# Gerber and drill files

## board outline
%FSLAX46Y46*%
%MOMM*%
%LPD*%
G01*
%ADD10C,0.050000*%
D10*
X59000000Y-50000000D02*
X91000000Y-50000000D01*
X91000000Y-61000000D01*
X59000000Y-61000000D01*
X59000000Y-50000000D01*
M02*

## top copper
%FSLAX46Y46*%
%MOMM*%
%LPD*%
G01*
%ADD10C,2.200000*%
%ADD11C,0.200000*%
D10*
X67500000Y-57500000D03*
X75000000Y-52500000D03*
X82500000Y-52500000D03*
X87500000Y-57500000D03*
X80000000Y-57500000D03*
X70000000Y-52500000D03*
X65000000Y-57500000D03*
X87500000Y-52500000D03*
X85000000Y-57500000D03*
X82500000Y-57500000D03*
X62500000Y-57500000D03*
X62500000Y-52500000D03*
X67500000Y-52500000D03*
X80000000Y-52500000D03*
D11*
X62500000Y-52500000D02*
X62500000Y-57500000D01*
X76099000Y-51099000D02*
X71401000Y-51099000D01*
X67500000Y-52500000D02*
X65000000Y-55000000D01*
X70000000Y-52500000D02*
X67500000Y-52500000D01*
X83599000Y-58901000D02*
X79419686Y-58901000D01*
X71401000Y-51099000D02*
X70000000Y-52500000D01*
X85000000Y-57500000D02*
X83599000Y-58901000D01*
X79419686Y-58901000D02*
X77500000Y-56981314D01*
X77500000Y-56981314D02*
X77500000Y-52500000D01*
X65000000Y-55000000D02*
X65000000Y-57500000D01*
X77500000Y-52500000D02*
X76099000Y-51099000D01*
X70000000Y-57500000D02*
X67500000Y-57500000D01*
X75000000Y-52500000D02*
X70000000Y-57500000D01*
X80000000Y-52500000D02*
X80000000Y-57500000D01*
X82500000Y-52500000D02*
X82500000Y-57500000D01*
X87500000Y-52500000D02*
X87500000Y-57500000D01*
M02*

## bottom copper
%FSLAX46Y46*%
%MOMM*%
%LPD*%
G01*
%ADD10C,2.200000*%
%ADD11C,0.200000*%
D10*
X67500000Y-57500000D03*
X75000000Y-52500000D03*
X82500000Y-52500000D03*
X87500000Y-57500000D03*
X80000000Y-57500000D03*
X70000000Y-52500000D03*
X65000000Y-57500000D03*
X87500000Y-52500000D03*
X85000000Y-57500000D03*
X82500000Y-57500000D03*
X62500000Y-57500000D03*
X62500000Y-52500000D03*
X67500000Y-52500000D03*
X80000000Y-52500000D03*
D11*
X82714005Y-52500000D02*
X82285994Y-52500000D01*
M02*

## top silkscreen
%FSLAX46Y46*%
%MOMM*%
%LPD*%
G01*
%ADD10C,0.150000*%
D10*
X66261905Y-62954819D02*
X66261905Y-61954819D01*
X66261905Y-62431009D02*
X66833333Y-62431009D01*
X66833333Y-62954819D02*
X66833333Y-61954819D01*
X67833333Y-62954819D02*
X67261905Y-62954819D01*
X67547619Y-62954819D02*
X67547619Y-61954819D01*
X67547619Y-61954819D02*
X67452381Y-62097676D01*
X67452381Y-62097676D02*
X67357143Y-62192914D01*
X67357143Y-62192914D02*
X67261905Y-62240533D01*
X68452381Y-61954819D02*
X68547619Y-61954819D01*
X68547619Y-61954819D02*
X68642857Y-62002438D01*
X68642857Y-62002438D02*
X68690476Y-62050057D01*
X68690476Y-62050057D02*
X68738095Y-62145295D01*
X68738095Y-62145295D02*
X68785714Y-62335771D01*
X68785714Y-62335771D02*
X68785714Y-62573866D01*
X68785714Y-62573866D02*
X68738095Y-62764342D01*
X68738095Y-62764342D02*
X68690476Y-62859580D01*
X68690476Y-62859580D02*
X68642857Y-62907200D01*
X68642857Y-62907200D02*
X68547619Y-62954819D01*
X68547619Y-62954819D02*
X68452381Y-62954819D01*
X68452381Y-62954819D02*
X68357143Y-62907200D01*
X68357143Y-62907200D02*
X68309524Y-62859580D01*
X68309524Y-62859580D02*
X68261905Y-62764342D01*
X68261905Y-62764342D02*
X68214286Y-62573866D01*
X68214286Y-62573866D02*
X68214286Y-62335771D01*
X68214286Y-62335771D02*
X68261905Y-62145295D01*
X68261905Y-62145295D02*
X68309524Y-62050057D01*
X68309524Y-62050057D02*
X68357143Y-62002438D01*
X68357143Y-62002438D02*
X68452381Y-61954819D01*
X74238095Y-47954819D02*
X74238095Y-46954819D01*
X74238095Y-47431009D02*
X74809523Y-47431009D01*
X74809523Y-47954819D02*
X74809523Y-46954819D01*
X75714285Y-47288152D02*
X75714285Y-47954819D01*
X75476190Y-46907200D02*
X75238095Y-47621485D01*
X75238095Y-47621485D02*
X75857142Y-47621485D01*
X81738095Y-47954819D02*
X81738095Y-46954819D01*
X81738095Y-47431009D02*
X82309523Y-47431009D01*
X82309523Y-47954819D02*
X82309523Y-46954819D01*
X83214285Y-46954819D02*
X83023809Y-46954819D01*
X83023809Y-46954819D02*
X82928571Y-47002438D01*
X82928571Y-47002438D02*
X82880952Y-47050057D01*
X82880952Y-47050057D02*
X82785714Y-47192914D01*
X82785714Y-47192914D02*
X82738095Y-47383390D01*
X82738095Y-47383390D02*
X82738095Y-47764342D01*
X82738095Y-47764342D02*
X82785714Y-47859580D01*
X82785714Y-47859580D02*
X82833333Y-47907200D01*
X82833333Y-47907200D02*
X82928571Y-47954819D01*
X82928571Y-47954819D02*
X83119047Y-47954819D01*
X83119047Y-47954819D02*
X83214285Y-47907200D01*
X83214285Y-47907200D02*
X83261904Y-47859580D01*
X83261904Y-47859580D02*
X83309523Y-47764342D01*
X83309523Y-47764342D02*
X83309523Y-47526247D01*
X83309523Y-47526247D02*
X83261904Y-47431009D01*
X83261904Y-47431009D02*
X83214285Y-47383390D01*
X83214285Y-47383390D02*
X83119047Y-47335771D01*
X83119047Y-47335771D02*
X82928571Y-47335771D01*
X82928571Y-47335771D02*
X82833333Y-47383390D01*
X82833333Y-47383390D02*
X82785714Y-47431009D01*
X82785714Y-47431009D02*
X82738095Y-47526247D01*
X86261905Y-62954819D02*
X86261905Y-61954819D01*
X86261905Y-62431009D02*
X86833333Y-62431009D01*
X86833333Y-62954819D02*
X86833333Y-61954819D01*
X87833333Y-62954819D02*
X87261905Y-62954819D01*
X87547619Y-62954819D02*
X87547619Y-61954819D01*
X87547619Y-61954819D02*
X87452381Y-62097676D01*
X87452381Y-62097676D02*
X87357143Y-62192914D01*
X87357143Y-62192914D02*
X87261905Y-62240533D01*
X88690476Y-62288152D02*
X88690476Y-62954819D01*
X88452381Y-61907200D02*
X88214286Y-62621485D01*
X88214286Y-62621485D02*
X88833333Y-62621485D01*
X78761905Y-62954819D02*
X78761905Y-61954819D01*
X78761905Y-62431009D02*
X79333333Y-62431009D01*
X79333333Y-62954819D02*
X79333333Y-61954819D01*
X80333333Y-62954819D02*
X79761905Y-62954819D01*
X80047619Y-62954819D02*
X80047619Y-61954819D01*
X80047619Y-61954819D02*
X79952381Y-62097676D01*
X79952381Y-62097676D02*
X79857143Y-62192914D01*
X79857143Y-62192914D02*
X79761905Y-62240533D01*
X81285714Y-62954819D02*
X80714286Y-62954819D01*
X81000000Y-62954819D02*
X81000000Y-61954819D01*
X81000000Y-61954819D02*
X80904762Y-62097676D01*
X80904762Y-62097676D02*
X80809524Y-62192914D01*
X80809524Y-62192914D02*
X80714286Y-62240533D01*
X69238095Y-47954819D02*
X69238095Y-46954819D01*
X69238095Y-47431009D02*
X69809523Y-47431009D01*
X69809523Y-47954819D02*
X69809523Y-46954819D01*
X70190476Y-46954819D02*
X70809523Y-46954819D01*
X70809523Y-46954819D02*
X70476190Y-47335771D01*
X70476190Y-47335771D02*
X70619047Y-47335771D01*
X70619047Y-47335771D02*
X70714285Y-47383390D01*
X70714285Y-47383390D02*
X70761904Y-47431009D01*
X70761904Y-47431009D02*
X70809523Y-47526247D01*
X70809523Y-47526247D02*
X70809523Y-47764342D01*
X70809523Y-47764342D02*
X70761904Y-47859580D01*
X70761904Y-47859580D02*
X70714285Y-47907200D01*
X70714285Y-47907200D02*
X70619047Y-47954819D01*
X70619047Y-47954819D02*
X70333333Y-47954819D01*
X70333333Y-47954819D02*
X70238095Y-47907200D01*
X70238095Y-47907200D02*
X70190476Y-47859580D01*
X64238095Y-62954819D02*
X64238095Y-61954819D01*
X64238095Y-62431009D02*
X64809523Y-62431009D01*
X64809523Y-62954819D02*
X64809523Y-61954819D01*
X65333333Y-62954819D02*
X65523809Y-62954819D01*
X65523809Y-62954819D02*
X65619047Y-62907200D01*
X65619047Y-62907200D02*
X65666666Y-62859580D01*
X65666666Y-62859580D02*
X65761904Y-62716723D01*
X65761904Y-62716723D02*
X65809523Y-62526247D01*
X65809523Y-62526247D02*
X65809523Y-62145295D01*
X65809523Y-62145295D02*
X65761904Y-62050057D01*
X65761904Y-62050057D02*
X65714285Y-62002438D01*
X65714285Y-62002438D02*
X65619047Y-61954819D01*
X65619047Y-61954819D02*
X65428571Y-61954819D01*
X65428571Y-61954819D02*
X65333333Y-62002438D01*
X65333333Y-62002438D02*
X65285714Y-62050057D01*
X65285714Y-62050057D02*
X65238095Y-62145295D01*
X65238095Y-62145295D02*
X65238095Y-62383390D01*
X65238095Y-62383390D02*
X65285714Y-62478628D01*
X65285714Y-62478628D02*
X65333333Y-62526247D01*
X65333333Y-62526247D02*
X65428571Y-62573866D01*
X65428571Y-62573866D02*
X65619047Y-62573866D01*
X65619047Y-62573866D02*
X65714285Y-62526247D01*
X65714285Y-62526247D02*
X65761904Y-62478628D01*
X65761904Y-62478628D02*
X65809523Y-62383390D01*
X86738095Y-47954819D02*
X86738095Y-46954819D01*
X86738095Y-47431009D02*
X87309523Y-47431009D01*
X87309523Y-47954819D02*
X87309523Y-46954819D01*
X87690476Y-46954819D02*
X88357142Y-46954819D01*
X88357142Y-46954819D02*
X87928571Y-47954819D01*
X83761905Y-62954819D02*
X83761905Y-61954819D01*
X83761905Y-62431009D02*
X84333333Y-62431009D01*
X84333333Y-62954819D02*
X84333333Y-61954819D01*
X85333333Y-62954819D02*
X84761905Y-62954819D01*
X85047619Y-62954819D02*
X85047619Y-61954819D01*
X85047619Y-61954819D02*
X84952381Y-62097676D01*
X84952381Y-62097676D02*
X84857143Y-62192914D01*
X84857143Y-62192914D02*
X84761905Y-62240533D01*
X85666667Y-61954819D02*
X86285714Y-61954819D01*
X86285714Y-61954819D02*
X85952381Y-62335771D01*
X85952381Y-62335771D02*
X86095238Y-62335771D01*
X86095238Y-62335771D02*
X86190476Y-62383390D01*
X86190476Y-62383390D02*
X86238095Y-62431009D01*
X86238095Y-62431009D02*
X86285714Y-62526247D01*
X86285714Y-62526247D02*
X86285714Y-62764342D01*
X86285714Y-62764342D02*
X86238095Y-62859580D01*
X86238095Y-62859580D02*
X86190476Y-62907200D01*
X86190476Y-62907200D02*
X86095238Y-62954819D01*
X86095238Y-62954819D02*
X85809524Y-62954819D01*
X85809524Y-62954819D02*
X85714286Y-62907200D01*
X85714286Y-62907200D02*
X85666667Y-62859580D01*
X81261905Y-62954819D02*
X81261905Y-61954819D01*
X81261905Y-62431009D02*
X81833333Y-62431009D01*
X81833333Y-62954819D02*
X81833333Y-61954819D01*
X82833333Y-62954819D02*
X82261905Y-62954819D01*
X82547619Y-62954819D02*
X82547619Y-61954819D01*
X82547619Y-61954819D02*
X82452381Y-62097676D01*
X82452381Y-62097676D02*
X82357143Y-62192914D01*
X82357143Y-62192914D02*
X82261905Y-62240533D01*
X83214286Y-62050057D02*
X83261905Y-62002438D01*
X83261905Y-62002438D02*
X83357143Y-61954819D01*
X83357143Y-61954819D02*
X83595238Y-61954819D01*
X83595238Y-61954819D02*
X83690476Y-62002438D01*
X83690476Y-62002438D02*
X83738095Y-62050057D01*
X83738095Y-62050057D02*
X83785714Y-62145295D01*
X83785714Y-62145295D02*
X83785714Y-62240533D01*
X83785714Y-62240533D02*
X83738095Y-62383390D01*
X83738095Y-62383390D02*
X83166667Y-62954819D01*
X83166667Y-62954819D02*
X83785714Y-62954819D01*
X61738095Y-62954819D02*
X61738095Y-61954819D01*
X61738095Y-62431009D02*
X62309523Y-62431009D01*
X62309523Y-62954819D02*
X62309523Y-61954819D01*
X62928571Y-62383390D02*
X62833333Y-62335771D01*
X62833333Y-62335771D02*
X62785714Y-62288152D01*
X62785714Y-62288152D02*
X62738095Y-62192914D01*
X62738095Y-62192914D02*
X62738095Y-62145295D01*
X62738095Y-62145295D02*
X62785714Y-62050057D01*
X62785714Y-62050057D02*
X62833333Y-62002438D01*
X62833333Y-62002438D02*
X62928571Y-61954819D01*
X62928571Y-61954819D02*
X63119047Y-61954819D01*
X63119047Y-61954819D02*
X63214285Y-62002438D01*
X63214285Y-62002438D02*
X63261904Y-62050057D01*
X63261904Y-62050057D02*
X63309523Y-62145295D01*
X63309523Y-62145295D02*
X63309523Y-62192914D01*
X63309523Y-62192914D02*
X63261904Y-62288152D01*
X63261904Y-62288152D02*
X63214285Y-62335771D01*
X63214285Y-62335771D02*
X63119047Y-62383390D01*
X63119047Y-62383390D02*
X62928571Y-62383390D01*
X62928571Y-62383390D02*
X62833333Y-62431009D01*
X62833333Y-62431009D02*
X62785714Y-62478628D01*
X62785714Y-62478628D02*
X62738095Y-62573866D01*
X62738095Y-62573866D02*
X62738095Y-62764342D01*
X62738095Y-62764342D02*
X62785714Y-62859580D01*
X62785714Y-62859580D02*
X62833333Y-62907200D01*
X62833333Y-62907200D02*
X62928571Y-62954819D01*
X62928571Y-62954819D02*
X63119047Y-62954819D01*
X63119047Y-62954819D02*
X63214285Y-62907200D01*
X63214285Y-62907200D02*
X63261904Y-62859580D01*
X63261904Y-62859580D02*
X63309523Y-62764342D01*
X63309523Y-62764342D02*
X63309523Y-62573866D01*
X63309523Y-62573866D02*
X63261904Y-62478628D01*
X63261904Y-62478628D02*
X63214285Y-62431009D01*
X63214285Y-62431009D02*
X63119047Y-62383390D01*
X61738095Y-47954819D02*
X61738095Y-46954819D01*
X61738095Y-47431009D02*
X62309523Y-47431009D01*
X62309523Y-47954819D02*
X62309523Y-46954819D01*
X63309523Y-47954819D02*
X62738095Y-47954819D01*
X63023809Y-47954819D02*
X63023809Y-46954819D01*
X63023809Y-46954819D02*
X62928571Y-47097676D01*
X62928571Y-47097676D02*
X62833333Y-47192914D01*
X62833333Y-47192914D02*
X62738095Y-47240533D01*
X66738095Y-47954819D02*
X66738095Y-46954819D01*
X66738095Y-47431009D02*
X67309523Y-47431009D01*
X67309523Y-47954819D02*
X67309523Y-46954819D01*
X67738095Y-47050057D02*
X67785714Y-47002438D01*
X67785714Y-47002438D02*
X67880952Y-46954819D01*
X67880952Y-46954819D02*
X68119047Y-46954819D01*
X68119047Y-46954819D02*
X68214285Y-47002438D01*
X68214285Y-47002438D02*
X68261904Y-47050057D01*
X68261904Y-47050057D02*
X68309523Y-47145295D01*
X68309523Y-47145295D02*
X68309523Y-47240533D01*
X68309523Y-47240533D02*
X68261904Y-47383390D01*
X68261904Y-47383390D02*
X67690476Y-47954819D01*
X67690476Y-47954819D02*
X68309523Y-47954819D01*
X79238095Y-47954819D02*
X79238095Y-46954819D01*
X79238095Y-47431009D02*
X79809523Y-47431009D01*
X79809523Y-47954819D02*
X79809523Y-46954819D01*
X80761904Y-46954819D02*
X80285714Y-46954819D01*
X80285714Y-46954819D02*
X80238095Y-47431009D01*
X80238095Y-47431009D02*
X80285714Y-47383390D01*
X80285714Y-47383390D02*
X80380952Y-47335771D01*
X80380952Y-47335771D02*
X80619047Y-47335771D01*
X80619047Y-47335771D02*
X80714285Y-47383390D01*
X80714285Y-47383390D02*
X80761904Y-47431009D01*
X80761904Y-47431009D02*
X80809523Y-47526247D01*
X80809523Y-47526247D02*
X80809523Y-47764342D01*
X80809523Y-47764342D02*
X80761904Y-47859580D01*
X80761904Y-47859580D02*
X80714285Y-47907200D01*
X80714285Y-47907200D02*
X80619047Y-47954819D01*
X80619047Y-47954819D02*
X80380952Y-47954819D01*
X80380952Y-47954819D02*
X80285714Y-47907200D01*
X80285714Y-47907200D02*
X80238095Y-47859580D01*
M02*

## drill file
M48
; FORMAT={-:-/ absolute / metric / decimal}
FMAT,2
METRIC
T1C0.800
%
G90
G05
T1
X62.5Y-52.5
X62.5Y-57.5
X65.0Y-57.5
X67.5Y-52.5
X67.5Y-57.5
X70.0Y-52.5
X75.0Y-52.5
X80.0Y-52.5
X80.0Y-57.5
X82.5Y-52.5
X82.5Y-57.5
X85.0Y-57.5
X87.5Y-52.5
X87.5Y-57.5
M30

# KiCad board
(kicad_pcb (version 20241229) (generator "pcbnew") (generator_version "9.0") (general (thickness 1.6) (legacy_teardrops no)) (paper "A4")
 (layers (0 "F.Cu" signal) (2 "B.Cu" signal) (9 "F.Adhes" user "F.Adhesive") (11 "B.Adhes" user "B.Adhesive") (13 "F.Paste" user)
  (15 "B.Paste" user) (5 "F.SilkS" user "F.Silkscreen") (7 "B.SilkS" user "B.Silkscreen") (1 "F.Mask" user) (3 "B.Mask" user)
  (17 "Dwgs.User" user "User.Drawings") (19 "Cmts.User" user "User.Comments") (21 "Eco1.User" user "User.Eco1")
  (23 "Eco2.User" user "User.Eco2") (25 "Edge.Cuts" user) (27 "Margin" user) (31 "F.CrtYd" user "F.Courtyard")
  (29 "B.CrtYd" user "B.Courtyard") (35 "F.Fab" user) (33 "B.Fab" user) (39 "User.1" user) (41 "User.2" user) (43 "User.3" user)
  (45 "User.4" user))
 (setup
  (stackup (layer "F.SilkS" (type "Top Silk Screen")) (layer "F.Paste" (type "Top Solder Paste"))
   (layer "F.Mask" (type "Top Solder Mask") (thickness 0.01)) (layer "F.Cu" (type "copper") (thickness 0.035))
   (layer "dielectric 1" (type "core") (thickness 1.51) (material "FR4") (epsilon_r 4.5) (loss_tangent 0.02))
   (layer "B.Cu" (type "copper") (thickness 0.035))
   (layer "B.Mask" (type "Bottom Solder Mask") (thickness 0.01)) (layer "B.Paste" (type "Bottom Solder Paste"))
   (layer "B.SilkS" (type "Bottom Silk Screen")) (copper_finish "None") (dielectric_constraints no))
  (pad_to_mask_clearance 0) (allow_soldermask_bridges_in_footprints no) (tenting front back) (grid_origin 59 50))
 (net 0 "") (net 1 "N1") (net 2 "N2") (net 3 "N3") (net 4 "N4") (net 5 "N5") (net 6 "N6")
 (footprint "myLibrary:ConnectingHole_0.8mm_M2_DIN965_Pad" (layer "F.Cu") (at 67.5 57.5)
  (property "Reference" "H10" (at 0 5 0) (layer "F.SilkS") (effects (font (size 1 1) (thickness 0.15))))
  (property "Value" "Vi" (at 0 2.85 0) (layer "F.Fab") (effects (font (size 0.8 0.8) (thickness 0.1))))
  (pad "1" thru_hole circle (at 0 0) (size 2.2 2.2) (drill 0.8) (layers "*.Cu" "*.Mask") (remove_unused_layers no) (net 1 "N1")
   (zone_connect 2)))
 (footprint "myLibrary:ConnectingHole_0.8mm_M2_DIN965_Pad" (layer "F.Cu") (at 75 52.5)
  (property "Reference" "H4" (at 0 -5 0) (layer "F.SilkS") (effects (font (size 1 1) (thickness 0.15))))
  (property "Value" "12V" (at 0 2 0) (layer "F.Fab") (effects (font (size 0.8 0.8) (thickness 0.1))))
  (pad "1" thru_hole circle (at 0 0) (size 2.2 2.2) (drill 0.8) (layers "*.Cu" "*.Mask") (remove_unused_layers no) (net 1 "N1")
   (zone_connect 2)))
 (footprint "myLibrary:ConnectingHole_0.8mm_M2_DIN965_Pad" (layer "F.Cu") (at 82.5 52.5)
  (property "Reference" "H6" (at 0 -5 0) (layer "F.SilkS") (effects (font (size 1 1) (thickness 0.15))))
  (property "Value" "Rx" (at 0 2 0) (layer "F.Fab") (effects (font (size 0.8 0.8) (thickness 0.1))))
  (pad "1" thru_hole circle (at 0 0) (size 2.2 2.2) (drill 0.8) (layers "*.Cu" "*.Mask") (remove_unused_layers no) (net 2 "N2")
   (zone_connect 2)))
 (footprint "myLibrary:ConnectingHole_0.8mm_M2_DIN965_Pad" (layer "F.Cu") (at 87.5 57.5)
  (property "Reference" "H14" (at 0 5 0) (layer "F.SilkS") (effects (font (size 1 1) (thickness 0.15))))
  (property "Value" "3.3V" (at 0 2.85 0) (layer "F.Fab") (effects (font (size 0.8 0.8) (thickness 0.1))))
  (pad "1" thru_hole circle (at 0 0) (size 2.2 2.2) (drill 0.8) (layers "*.Cu" "*.Mask") (remove_unused_layers no) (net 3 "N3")
   (zone_connect 2)))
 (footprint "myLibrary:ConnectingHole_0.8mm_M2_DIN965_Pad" (layer "F.Cu") (at 80 57.5)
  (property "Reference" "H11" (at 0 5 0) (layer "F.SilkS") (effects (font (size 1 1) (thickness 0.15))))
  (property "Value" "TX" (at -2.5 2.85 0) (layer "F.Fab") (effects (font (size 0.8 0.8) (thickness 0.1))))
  (pad "1" thru_hole circle (at 0 0) (size 2.2 2.2) (drill 0.8) (layers "*.Cu" "*.Mask") (remove_unused_layers no) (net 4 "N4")
   (zone_connect 2)))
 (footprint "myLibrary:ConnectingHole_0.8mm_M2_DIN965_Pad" (layer "F.Cu") (at 70 52.5)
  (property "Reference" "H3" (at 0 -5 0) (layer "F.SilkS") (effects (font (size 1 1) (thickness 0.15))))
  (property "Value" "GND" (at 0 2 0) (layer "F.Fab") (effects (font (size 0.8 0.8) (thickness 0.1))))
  (pad "1" thru_hole circle (at 0 0) (size 2.2 2.2) (drill 0.8) (layers "*.Cu" "*.Mask") (remove_unused_layers no) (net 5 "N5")
   (zone_connect 2)))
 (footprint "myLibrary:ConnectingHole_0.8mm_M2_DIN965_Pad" (layer "F.Cu") (at 65 57.5)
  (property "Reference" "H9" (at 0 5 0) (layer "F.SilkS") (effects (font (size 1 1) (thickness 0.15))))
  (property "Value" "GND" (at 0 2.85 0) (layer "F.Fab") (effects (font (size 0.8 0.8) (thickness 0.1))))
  (pad "1" thru_hole circle (at 0 0) (size 2.2 2.2) (drill 0.8) (layers "*.Cu" "*.Mask") (remove_unused_layers no) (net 5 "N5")
   (zone_connect 2)))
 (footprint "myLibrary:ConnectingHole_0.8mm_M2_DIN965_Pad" (layer "F.Cu") (at 87.5 52.5)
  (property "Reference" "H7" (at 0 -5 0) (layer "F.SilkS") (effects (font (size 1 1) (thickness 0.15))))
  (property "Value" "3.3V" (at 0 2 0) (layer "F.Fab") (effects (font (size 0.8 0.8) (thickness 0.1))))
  (pad "1" thru_hole circle (at 0 0) (size 2.2 2.2) (drill 0.8) (layers "*.Cu" "*.Mask") (remove_unused_layers no) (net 3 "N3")
   (zone_connect 2)))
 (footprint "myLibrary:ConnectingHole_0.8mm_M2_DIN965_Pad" (layer "F.Cu") (at 85 57.5)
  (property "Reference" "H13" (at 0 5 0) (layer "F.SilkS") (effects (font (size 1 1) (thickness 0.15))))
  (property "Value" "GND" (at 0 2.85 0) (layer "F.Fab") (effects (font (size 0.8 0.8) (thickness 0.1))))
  (pad "1" thru_hole circle (at 0 0) (size 2.2 2.2) (drill 0.8) (layers "*.Cu" "*.Mask") (remove_unused_layers no) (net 5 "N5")
   (zone_connect 2)))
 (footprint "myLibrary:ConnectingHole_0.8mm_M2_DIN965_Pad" (layer "F.Cu") (at 82.5 57.5)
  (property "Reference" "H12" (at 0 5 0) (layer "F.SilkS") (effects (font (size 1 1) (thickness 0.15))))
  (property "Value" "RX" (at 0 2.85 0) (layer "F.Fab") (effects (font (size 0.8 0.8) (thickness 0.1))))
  (pad "1" thru_hole circle (at 0 0) (size 2.2 2.2) (drill 0.8) (layers "*.Cu" "*.Mask") (remove_unused_layers no) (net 2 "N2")
   (zone_connect 2)))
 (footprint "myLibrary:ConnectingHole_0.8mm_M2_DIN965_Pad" (layer "F.Cu") (at 62.5 57.5)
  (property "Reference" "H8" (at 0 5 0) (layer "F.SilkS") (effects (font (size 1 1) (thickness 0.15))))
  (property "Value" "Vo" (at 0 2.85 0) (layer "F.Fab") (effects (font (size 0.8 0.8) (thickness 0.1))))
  (pad "1" thru_hole circle (at 0 0) (size 2.2 2.2) (drill 0.8) (layers "*.Cu" "*.Mask") (remove_unused_layers no) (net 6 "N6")
   (zone_connect 2)))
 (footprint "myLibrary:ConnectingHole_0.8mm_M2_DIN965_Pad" (layer "F.Cu") (at 62.5 52.5)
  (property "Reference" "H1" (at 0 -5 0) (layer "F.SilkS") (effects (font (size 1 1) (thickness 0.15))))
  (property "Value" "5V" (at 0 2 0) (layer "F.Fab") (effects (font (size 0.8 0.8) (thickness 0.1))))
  (pad "1" thru_hole circle (at 0 0) (size 2.2 2.2) (drill 0.8) (layers "*.Cu" "*.Mask") (remove_unused_layers no) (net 6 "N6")
   (zone_connect 2)))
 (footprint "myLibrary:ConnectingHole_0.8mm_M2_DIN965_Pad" (layer "F.Cu") (at 67.5 52.5)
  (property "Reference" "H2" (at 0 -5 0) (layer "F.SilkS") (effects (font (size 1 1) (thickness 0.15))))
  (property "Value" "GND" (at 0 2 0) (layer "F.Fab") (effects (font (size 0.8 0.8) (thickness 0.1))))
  (pad "1" thru_hole circle (at 0 0) (size 2.2 2.2) (drill 0.8) (layers "*.Cu" "*.Mask") (remove_unused_layers no) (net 5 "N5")
   (zone_connect 2)))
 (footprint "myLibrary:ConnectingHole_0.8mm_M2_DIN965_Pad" (layer "F.Cu") (at 80 52.5)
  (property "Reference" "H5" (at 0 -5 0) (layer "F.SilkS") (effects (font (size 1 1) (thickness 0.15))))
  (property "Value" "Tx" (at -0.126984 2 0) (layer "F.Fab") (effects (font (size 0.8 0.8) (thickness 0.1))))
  (pad "1" thru_hole circle (at 0 0) (size 2.2 2.2) (drill 0.8) (layers "*.Cu" "*.Mask") (remove_unused_layers no) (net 4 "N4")
   (zone_connect 2)))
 (gr_rect (start 59 50) (end 91 61) (stroke (width 0.05) (type solid)) (fill no) (layer "Edge.Cuts"))
 (segment (start 62.5 52.5) (end 62.5 57.5) (width 0.2) (layer "F.Cu") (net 6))
 (segment (start 76.099 51.099) (end 71.401 51.099) (width 0.2) (layer "F.Cu") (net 5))
 (segment (start 67.5 52.5) (end 65 55) (width 0.2) (layer "F.Cu") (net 5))
 (segment (start 70 52.5) (end 67.5 52.5) (width 0.2) (layer "F.Cu") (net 5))
 (segment (start 83.599 58.901) (end 79.419686 58.901) (width 0.2) (layer "F.Cu") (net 5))
 (segment (start 71.401 51.099) (end 70 52.5) (width 0.2) (layer "F.Cu") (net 5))
 (segment (start 85 57.5) (end 83.599 58.901) (width 0.2) (layer "F.Cu") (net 5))
 (segment (start 79.419686 58.901) (end 77.5 56.981314) (width 0.2) (layer "F.Cu") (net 5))
 (segment (start 77.5 56.981314) (end 77.5 52.5) (width 0.2) (layer "F.Cu") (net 5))
 (segment (start 65 55) (end 65 57.5) (width 0.2) (layer "F.Cu") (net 5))
 (segment (start 77.5 52.5) (end 76.099 51.099) (width 0.2) (layer "F.Cu") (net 5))
 (segment (start 70 57.5) (end 67.5 57.5) (width 0.2) (layer "F.Cu") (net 1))
 (segment (start 75 52.5) (end 70 57.5) (width 0.2) (layer "F.Cu") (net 1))
 (segment (start 80 52.5) (end 80 57.5) (width 0.2) (layer "F.Cu") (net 4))
 (segment (start 82.5 52.5) (end 82.5 57.5) (width 0.2) (layer "F.Cu") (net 2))
 (segment (start 82.714005 52.5) (end 82.285994 52.5) (width 0.2) (layer "B.Cu") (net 2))
 (segment (start 87.5 52.5) (end 87.5 57.5) (width 0.2) (layer "F.Cu") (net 3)))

